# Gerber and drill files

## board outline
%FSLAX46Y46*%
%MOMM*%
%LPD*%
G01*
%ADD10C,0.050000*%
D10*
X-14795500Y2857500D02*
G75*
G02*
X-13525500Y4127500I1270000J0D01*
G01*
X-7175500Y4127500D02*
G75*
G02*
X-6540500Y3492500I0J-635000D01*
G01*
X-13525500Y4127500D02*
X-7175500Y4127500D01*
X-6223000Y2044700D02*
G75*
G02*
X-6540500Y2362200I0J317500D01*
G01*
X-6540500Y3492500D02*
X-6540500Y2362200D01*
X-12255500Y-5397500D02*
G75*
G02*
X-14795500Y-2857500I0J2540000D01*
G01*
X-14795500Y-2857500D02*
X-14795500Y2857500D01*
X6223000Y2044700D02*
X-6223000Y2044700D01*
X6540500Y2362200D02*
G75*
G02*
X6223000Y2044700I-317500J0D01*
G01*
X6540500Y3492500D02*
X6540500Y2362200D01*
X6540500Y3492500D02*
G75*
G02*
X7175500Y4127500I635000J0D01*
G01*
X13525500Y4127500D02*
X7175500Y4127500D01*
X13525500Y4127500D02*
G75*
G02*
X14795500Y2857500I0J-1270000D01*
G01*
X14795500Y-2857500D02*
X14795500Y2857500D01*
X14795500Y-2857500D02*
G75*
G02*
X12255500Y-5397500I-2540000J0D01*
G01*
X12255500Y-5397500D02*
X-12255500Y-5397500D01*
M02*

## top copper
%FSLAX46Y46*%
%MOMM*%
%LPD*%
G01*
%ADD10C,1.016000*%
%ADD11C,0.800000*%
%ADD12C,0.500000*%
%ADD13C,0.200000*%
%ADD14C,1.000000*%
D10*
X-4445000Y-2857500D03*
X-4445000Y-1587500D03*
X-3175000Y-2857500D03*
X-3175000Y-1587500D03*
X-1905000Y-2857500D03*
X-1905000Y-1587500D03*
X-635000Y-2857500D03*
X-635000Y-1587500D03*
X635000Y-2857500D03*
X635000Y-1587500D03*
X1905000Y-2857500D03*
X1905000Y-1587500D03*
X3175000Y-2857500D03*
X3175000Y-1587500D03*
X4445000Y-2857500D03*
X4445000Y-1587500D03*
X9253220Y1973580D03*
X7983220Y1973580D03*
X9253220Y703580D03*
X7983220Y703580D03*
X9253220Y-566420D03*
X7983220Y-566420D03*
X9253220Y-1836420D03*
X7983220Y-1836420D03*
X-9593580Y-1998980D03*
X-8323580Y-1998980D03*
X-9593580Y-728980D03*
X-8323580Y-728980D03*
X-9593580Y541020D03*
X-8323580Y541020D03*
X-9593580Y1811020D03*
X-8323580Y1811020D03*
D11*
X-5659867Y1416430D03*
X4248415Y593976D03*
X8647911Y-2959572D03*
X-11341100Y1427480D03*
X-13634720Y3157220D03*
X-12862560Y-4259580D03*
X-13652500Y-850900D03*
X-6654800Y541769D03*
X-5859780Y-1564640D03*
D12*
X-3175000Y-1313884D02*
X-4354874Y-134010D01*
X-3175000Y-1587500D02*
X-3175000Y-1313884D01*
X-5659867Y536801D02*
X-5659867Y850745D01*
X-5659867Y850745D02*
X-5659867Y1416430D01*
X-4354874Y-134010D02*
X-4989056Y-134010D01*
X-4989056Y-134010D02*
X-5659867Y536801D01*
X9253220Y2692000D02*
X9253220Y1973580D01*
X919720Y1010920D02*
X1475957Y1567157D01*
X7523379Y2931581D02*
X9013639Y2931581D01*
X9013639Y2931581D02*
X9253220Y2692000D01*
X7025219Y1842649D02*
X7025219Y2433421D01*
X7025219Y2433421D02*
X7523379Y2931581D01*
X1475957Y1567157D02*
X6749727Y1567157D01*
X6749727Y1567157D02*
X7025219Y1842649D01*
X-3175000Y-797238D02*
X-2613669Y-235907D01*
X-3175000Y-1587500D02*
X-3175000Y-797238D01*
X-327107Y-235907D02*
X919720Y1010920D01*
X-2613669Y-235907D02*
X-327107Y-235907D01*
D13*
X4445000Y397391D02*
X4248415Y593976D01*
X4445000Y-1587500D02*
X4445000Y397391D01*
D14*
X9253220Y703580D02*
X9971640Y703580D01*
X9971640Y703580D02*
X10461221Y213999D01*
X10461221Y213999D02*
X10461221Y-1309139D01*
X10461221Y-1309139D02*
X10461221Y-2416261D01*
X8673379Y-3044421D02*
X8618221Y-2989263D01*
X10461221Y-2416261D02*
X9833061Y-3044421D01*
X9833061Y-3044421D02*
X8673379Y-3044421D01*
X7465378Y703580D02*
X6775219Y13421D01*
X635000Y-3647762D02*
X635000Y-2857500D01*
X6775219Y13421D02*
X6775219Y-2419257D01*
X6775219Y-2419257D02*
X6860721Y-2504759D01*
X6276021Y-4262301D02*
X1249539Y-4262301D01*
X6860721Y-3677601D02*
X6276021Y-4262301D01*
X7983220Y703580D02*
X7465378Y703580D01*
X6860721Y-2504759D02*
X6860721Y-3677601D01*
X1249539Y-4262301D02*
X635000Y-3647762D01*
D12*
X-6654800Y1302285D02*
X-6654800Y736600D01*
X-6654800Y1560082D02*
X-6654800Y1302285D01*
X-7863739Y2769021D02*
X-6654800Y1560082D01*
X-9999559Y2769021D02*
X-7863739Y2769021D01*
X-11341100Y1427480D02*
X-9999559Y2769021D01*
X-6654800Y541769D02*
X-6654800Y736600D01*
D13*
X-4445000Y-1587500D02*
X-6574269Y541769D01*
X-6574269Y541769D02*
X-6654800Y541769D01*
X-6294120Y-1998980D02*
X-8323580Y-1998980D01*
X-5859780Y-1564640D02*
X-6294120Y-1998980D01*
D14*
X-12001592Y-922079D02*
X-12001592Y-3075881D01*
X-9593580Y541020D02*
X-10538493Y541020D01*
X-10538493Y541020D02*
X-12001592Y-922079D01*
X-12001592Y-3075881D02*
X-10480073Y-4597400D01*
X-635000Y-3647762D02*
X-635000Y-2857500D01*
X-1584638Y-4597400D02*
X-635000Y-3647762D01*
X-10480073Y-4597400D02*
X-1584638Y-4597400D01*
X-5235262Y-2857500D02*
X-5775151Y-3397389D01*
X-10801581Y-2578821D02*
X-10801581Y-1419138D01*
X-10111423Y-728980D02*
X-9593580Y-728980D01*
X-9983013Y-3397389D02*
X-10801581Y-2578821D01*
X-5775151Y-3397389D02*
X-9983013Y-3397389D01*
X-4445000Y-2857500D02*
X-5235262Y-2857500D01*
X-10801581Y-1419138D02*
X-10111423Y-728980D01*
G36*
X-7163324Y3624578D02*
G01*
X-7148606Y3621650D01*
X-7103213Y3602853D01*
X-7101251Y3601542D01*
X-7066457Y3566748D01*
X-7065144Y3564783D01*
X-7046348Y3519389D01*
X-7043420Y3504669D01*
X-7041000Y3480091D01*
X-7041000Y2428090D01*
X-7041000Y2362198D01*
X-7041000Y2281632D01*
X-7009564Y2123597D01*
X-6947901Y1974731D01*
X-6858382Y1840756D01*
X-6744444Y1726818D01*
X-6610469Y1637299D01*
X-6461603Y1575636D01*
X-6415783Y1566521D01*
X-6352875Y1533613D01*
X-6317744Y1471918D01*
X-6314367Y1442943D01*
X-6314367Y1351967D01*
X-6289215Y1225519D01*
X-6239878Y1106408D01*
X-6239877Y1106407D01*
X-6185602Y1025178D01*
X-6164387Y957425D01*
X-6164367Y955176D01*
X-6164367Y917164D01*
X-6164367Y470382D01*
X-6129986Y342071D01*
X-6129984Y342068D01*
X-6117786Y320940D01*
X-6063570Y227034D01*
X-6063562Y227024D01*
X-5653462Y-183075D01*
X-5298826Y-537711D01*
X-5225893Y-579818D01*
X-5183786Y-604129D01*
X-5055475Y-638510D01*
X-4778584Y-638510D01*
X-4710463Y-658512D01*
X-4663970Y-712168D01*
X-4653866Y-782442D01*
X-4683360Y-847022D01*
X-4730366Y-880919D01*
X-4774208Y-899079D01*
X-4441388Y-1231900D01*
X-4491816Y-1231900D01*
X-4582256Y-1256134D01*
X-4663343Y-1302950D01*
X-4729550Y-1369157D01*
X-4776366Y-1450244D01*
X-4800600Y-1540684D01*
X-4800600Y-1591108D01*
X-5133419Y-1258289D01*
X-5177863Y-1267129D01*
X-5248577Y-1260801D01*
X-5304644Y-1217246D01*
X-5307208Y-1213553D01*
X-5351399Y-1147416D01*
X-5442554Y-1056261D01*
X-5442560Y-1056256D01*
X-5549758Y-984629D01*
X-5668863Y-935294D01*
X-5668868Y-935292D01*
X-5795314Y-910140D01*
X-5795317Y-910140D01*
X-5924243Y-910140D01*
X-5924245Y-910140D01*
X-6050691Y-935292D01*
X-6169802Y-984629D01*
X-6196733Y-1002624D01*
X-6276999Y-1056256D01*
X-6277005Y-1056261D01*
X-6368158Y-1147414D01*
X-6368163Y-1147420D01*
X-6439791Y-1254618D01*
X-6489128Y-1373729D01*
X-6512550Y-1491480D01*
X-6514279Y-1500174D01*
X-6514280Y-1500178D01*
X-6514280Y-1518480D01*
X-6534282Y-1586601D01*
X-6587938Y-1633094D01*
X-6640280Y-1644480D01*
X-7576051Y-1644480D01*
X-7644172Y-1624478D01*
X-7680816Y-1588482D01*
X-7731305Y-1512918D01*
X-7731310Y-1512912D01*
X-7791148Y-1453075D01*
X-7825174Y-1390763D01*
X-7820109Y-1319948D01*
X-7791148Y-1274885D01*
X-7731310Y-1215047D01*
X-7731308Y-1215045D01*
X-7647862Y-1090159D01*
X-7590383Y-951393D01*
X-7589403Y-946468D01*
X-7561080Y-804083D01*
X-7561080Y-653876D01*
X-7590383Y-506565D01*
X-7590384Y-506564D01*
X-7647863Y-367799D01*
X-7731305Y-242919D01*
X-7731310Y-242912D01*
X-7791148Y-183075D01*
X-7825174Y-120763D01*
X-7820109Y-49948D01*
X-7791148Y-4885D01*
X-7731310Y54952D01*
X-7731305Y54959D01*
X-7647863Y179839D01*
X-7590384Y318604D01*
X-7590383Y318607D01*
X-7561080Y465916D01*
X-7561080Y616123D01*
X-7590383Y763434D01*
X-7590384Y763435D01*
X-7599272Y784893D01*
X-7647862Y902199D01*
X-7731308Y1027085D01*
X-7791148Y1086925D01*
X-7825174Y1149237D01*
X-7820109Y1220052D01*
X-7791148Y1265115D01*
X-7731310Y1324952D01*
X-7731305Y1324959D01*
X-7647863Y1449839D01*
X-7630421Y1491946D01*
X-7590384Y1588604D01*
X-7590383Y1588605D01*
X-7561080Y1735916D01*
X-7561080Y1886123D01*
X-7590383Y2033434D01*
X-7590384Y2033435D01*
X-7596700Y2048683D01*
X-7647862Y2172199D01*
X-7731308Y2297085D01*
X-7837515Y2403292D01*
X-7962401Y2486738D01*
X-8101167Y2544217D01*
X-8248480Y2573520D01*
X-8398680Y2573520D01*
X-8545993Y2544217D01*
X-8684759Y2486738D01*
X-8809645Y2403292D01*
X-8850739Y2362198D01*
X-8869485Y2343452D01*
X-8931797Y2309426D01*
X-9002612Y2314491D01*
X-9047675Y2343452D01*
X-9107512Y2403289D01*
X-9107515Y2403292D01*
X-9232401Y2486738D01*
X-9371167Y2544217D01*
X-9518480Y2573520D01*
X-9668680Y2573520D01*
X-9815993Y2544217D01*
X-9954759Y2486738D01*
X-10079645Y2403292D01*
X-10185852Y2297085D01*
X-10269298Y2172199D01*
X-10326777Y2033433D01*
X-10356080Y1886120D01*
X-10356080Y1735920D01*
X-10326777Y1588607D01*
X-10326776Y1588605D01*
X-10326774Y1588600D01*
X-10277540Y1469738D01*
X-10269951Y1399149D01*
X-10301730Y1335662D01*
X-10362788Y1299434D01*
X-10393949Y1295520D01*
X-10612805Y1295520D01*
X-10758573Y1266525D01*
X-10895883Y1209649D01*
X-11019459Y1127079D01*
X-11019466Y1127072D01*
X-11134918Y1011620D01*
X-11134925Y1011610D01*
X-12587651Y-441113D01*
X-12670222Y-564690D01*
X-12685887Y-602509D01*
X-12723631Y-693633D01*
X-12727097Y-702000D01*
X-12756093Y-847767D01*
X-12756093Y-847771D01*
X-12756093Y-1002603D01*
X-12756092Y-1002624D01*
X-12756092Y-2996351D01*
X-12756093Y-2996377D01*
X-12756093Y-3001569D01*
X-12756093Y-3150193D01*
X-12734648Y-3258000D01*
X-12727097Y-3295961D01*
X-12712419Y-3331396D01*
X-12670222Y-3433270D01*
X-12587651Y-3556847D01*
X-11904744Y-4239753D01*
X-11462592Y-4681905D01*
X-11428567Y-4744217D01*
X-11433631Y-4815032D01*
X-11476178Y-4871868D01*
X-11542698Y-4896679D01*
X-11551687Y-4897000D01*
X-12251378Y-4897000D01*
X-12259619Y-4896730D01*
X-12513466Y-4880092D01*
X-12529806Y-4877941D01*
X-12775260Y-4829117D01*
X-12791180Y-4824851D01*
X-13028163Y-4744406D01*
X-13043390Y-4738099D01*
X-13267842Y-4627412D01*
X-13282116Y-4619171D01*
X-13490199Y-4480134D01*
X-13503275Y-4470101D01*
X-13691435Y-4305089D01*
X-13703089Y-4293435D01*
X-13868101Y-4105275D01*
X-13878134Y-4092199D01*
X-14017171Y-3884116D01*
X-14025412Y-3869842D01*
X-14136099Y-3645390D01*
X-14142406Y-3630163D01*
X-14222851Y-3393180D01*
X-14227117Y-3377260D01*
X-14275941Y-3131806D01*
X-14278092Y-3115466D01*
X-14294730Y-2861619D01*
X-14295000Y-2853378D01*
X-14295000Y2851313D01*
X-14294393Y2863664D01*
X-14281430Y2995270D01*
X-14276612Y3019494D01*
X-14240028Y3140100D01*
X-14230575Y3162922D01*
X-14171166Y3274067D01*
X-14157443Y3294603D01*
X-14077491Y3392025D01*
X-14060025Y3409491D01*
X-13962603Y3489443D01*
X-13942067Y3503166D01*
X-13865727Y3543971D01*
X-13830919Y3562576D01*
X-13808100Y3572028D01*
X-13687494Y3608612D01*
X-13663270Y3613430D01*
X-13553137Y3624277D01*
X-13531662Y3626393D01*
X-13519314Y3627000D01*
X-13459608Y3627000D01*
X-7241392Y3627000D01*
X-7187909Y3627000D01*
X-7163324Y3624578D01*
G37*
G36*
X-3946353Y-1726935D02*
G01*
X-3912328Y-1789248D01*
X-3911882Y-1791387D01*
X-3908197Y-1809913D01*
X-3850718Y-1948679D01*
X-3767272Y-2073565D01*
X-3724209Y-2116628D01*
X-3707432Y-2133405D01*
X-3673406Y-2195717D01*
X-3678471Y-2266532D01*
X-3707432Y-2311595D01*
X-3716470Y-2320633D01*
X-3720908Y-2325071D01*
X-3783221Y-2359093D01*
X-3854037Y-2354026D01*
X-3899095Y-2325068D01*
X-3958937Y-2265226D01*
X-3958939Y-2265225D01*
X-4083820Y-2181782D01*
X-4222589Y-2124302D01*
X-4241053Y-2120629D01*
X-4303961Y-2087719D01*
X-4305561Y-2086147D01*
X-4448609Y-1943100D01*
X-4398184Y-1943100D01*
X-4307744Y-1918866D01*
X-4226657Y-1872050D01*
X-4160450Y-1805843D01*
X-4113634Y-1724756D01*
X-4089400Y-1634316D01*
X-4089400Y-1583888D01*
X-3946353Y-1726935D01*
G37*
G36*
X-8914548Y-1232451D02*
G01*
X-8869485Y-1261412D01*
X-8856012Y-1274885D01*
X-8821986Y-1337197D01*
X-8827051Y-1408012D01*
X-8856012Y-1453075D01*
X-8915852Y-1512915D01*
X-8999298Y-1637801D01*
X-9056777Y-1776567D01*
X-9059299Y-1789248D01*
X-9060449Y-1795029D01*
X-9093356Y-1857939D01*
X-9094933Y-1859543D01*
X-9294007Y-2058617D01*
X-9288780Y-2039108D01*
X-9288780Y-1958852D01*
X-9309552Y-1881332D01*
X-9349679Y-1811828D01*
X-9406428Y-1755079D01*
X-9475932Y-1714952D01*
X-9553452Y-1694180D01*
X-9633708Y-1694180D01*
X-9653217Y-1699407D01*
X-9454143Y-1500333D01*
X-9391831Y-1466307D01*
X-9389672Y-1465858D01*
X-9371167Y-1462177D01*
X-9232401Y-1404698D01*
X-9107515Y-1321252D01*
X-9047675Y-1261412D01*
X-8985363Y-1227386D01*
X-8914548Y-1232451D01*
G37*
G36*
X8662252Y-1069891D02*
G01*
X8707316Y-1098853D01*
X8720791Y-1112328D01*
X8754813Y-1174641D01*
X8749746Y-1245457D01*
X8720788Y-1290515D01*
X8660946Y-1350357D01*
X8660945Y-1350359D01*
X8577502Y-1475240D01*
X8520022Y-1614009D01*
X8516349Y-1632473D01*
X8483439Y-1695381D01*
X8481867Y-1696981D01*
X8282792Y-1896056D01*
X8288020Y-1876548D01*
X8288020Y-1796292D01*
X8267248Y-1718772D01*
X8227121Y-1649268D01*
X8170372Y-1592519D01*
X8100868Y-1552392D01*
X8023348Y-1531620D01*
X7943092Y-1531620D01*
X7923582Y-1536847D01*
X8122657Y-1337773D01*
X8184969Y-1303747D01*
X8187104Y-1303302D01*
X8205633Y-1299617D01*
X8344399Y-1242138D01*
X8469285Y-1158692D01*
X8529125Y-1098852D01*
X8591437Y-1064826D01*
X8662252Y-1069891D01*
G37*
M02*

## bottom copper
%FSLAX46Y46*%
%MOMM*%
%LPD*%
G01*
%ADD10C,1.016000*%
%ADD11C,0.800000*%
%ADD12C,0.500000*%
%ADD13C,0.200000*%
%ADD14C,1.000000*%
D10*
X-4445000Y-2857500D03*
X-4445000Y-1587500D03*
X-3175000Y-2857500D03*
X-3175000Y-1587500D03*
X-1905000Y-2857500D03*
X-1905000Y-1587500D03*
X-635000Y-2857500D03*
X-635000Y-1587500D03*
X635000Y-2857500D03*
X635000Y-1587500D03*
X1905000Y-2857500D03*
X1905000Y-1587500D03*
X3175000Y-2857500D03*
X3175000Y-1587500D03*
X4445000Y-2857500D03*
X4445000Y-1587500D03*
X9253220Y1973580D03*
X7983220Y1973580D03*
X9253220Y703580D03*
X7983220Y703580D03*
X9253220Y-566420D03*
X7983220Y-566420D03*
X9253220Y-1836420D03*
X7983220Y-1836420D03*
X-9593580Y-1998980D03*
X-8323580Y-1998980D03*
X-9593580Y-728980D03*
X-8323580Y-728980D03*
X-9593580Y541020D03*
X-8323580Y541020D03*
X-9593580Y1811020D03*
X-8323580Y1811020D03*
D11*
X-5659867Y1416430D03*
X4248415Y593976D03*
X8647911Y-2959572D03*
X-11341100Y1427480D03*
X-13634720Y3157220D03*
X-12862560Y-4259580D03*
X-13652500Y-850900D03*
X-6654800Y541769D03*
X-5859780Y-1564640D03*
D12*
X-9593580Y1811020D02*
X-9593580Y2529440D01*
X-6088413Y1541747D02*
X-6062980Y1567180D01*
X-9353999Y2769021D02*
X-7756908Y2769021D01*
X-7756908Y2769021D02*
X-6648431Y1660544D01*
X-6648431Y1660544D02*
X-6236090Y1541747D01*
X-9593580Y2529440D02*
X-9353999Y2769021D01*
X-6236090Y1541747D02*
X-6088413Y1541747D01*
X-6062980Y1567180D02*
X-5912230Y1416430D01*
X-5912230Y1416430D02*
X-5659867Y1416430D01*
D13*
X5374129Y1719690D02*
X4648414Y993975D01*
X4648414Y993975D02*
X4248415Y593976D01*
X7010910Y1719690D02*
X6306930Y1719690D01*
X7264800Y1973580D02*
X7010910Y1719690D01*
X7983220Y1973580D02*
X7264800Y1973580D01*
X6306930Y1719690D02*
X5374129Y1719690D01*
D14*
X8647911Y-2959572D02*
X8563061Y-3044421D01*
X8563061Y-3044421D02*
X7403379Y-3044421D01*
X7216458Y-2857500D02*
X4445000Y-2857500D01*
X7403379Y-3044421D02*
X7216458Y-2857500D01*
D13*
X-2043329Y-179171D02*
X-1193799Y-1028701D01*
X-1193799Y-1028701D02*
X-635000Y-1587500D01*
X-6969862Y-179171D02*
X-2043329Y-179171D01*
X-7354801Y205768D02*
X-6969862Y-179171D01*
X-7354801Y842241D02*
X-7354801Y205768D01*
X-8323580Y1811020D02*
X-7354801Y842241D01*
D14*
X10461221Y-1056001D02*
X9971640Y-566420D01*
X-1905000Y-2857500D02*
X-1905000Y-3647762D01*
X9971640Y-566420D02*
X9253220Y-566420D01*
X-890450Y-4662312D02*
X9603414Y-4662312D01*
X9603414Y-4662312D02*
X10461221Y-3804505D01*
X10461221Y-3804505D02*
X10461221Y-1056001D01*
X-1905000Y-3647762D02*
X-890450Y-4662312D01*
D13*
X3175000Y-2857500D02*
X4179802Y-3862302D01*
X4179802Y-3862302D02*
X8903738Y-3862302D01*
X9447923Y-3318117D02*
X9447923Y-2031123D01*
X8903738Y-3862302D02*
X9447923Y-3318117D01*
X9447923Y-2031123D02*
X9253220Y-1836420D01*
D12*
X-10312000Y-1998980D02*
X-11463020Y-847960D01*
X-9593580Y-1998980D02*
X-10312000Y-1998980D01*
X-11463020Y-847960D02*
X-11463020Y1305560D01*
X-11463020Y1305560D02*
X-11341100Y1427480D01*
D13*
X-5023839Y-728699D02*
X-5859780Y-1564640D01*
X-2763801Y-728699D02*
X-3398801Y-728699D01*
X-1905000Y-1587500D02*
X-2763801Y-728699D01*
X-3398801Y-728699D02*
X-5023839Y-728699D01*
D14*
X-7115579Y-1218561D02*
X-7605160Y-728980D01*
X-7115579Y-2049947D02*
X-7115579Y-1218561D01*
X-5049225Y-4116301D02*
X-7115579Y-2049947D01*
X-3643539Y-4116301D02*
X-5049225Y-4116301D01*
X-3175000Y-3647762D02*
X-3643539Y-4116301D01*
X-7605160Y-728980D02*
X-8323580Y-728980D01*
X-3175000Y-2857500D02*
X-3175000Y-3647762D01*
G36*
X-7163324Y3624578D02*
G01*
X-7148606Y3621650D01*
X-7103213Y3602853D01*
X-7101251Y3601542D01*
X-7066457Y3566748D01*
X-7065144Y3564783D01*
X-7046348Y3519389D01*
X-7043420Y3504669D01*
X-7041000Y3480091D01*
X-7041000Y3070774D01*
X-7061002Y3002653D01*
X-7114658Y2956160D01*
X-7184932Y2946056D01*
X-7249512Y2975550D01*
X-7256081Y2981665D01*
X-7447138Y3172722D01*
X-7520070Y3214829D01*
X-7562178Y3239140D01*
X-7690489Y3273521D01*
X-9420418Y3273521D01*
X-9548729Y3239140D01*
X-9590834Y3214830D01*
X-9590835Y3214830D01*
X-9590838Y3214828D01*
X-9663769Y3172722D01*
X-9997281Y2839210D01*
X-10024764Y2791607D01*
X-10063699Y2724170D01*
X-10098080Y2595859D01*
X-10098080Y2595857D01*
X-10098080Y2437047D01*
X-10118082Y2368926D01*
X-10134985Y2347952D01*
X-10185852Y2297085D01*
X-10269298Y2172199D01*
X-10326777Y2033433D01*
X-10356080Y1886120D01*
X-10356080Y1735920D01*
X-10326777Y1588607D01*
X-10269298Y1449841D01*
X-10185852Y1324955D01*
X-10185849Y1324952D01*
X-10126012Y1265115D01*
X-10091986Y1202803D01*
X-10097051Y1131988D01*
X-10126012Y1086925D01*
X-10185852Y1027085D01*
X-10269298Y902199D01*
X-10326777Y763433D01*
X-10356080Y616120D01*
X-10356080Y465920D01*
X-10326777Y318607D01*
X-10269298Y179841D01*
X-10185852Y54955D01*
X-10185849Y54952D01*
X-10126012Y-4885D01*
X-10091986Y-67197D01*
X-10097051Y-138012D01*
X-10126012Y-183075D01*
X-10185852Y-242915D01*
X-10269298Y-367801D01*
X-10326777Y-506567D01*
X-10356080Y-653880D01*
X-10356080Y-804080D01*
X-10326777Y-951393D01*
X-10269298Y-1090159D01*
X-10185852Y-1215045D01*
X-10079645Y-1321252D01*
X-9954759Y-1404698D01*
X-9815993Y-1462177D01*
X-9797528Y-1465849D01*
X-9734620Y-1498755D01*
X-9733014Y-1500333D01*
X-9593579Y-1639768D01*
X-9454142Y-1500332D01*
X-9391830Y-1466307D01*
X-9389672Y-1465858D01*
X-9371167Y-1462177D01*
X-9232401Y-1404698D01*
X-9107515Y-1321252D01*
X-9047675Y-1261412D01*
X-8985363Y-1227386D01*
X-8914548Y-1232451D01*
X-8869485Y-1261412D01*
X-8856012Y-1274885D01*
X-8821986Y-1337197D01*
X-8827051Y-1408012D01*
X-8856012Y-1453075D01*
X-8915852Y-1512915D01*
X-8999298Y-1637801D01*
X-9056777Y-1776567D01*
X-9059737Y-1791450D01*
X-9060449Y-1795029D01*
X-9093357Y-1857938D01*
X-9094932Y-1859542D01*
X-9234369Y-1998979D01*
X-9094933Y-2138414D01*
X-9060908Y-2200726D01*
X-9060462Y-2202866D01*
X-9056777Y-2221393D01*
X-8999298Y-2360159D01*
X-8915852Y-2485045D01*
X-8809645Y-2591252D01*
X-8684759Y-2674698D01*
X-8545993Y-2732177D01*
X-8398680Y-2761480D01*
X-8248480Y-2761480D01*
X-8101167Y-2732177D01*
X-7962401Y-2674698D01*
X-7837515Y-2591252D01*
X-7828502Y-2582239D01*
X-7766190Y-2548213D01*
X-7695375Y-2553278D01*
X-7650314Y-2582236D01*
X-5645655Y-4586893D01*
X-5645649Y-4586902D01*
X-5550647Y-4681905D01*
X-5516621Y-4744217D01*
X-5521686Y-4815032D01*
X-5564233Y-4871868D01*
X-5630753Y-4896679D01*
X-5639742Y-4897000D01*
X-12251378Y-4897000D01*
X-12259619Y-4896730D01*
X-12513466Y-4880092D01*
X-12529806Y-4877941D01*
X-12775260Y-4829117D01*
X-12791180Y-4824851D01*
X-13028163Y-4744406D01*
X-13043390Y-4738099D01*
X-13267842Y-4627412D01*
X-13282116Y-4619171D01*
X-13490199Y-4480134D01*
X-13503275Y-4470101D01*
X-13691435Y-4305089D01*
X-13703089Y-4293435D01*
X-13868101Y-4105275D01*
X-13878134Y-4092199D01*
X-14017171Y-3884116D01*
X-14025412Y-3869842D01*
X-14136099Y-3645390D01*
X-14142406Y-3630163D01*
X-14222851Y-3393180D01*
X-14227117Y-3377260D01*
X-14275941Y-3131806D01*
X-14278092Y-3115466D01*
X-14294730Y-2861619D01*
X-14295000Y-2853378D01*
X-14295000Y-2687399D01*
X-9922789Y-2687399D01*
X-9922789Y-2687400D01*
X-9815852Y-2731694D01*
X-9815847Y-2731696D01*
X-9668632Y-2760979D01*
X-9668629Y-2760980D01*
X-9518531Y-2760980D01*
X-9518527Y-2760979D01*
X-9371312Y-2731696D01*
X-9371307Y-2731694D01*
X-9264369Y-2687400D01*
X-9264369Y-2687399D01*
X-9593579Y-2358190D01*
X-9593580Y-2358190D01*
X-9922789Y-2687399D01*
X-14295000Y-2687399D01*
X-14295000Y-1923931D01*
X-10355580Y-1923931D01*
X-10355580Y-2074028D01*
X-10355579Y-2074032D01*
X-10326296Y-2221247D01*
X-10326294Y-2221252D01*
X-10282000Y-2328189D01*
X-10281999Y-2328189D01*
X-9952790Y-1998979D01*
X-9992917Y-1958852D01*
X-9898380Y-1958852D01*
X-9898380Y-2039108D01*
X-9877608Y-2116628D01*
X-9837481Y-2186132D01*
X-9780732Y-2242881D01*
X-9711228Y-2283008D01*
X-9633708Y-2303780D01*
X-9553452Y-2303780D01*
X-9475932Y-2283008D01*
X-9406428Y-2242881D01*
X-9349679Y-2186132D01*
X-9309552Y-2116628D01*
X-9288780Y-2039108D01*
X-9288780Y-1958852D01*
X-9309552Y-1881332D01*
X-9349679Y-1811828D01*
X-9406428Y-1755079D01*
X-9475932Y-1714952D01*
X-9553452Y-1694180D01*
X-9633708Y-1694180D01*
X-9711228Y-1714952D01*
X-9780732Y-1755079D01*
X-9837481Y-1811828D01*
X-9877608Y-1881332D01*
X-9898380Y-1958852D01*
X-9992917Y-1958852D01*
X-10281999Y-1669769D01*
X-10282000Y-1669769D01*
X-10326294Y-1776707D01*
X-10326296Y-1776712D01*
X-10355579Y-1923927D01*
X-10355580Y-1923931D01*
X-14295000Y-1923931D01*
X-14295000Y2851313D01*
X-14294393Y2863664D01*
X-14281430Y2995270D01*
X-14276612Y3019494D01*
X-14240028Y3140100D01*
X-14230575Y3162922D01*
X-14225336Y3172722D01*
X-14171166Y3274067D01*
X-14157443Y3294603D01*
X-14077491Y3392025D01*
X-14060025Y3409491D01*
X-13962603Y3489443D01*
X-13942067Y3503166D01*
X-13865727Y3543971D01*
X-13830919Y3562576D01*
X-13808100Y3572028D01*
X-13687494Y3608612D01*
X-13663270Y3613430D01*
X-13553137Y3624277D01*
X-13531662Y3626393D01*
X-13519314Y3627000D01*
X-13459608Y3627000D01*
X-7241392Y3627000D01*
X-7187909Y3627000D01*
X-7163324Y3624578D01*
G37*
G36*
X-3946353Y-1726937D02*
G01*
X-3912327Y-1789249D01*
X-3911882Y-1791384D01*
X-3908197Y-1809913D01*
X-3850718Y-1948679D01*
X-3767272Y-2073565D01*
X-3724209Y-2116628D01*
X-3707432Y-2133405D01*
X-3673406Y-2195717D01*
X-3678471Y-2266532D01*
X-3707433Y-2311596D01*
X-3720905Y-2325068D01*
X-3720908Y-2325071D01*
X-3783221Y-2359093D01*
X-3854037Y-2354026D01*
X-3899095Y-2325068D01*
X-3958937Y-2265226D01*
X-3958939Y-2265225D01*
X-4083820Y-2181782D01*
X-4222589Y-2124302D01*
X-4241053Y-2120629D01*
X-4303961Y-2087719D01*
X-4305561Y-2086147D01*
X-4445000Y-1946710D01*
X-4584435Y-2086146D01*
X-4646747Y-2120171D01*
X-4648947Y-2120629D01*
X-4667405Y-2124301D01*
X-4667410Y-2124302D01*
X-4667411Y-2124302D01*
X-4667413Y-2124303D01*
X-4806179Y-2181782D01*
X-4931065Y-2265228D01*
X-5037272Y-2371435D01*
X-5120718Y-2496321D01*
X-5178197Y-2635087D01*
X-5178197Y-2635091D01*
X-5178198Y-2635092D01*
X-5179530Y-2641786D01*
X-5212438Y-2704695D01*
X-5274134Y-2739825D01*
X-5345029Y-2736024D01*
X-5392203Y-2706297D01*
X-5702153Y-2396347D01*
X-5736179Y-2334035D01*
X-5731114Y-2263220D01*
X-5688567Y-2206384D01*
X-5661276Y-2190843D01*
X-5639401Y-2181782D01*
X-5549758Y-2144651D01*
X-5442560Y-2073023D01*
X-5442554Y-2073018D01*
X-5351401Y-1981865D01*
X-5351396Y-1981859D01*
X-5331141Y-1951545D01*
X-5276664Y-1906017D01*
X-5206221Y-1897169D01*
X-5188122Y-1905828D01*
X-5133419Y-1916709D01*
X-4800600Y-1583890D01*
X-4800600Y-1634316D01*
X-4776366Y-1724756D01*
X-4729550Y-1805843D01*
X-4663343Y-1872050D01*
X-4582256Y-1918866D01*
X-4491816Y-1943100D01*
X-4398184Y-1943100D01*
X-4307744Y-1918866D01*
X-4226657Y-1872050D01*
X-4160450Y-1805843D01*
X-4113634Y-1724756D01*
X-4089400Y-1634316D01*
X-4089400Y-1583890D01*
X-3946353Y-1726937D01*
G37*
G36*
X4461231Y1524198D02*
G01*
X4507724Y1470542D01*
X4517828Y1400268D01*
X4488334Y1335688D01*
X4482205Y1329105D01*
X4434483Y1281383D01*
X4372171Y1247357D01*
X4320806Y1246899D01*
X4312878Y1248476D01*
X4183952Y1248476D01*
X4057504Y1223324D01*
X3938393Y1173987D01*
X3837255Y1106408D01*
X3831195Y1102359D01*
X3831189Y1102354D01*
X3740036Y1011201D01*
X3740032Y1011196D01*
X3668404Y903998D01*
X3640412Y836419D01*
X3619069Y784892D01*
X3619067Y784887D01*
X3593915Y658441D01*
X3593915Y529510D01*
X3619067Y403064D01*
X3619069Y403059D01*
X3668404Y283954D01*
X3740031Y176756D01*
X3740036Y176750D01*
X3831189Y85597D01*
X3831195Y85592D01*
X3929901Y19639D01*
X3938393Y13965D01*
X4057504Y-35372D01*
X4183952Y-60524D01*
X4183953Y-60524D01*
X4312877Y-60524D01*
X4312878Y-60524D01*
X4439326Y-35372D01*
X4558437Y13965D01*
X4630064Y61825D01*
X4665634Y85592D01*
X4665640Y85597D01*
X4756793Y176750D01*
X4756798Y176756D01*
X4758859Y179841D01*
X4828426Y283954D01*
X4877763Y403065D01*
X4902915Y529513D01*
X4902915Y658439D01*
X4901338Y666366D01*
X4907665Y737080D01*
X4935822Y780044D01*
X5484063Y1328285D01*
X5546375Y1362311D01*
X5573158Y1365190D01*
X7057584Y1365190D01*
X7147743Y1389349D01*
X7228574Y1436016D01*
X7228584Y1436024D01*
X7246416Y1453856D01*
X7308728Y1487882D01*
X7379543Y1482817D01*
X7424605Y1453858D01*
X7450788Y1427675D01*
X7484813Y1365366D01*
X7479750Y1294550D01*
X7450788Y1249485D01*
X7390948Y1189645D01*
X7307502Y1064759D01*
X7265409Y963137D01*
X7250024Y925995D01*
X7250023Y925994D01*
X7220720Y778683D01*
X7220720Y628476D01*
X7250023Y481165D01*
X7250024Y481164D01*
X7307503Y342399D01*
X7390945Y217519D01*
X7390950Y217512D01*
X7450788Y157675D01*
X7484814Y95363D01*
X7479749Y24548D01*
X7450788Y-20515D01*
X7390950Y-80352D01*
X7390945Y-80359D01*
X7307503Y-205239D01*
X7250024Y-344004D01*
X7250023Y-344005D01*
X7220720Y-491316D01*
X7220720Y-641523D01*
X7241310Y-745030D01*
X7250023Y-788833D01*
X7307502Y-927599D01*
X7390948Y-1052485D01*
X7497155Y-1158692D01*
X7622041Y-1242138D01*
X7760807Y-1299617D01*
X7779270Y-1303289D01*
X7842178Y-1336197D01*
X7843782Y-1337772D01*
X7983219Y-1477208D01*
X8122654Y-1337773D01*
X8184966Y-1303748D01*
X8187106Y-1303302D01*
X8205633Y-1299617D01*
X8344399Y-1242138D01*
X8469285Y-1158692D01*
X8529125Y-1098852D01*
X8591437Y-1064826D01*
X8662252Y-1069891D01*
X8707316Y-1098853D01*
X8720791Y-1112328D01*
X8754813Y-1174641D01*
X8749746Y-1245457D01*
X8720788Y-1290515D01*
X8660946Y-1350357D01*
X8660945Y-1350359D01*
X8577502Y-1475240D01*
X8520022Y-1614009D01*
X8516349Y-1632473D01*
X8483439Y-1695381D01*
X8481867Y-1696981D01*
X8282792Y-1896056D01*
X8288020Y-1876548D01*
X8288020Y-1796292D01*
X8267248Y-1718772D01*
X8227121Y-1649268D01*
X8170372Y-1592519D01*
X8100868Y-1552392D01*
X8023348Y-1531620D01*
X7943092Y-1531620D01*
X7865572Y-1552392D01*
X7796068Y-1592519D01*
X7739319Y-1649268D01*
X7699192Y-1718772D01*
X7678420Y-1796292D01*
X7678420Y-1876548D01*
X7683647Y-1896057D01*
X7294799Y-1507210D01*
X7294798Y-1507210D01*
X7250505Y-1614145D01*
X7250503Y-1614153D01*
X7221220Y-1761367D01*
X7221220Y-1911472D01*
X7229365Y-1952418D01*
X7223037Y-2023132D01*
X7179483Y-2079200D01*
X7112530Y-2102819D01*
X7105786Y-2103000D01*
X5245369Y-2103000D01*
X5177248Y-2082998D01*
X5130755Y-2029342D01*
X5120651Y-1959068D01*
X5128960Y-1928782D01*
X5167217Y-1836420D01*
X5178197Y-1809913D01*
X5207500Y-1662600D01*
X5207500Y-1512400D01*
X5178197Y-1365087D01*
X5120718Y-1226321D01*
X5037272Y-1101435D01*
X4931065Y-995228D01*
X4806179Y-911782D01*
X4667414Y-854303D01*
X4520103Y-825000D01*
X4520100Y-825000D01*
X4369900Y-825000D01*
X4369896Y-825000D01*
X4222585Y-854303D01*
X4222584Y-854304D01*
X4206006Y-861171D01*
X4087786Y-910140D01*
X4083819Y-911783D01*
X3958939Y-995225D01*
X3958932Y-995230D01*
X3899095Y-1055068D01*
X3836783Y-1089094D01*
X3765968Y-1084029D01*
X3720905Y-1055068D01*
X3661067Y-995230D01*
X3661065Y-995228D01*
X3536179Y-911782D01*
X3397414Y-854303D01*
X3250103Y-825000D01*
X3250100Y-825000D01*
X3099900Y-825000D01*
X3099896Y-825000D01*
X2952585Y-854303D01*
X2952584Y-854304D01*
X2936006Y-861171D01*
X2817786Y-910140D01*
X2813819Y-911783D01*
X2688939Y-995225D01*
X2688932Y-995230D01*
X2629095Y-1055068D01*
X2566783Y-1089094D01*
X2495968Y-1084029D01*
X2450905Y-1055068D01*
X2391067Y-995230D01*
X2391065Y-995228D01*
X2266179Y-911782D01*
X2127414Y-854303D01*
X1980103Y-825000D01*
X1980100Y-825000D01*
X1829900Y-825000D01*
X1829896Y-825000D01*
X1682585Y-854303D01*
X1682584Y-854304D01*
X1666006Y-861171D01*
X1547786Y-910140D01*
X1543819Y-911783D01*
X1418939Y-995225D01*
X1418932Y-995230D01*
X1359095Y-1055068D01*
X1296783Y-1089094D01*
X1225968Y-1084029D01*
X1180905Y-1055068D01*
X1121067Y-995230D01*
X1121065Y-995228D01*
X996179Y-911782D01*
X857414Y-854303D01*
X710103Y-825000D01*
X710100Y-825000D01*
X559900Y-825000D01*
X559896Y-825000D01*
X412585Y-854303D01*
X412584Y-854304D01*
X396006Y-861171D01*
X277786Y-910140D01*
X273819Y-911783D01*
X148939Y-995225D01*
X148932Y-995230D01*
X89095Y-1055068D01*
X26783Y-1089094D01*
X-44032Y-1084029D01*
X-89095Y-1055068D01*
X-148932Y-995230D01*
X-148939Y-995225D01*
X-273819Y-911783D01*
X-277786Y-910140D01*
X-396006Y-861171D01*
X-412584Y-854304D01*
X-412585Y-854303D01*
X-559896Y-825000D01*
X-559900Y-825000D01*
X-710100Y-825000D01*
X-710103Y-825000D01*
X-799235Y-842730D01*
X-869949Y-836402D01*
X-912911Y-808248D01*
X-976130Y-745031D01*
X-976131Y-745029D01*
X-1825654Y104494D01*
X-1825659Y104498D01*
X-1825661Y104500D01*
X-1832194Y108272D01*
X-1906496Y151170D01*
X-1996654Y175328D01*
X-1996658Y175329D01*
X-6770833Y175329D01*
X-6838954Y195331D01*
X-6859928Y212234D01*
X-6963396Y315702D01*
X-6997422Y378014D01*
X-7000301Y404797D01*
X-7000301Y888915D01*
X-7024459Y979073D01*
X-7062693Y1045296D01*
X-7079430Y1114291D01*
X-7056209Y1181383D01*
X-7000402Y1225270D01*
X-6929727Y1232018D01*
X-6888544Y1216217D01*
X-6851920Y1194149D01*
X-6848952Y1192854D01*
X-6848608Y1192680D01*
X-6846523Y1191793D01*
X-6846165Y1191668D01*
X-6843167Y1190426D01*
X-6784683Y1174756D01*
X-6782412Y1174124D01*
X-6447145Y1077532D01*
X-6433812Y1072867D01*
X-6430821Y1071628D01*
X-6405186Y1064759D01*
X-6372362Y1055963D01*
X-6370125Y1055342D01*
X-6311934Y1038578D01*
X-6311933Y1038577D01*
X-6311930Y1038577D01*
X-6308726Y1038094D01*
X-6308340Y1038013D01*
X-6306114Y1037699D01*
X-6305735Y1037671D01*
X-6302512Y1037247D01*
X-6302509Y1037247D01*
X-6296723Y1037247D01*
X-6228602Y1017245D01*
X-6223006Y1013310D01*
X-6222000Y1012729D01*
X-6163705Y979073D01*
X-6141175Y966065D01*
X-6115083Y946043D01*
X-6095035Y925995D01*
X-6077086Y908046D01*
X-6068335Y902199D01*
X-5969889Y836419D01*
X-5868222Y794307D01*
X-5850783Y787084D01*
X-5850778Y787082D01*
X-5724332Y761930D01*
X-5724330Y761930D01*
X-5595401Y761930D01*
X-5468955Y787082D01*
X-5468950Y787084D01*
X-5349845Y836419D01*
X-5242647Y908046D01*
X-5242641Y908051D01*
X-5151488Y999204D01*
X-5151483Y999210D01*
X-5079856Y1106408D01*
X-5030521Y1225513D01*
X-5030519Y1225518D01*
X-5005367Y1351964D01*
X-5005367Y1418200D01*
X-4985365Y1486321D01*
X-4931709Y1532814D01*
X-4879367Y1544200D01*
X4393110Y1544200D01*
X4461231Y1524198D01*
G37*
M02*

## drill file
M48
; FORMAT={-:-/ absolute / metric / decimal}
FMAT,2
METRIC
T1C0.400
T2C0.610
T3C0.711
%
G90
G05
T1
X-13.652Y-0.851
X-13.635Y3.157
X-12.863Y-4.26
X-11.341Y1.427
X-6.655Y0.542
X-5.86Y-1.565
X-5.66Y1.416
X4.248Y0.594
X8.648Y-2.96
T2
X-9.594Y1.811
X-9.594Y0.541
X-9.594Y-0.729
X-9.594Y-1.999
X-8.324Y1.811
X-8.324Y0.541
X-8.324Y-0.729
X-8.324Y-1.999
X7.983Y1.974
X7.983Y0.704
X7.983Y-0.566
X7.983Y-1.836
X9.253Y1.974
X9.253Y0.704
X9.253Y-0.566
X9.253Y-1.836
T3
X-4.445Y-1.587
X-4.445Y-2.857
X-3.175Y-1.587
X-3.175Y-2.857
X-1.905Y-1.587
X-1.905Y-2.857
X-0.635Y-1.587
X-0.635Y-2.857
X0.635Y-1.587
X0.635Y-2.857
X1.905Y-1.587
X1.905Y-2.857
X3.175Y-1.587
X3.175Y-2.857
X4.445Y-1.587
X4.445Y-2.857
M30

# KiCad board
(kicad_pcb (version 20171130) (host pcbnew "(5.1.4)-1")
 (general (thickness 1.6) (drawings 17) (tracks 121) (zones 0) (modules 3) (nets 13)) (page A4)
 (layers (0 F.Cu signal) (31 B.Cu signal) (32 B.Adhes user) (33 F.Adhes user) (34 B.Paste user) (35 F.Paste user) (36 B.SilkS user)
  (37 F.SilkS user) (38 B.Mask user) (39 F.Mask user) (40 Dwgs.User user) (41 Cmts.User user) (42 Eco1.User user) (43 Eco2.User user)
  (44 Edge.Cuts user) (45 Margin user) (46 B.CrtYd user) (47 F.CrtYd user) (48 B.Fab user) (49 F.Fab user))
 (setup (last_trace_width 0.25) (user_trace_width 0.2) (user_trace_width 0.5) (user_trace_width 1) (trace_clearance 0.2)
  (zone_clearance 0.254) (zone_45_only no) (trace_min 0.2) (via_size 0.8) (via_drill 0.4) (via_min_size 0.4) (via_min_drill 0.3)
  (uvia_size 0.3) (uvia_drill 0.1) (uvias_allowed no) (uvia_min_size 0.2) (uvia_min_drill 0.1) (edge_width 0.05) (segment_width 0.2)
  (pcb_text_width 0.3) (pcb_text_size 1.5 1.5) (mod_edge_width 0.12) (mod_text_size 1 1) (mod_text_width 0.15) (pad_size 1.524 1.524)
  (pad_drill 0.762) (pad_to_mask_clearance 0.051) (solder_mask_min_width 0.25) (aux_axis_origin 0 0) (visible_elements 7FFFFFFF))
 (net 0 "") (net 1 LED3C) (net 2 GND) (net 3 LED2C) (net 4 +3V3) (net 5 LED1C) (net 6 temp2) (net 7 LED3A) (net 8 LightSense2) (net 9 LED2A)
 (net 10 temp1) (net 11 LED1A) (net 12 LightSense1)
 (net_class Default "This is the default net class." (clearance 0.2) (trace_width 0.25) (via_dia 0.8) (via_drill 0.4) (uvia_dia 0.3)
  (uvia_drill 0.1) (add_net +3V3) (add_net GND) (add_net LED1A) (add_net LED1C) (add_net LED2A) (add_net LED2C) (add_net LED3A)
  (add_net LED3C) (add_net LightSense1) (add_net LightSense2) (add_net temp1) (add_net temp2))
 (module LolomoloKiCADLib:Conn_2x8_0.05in (layer F.Cu) (at 4.445 1.5875 270)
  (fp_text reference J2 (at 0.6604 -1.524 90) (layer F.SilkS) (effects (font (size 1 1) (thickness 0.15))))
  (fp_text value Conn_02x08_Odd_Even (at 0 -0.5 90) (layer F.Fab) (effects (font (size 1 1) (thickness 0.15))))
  (pad 16 thru_hole circle (at 1.27 8.89 270) (size 1.016 1.016) (drill 0.7112) (layers *.Cu *.Mask) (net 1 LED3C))
  (pad 15 thru_hole circle (at 0 8.89 270) (size 1.016 1.016) (drill 0.7112) (layers *.Cu *.Mask) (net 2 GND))
  (pad 14 thru_hole circle (at 1.27 7.62 270) (size 1.016 1.016) (drill 0.7112) (layers *.Cu *.Mask) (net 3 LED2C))
  (pad 13 thru_hole circle (at 0 7.62 270) (size 1.016 1.016) (drill 0.7112) (layers *.Cu *.Mask) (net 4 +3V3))
  (pad 12 thru_hole circle (at 1.27 6.35 270) (size 1.016 1.016) (drill 0.7112) (layers *.Cu *.Mask) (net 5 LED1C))
  (pad 11 thru_hole circle (at 0 6.35 270) (size 1.016 1.016) (drill 0.7112) (layers *.Cu *.Mask) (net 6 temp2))
  (pad 10 thru_hole circle (at 1.27 5.08 270) (size 1.016 1.016) (drill 0.7112) (layers *.Cu *.Mask) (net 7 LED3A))
  (pad 9 thru_hole circle (at 0 5.08 270) (size 1.016 1.016) (drill 0.7112) (layers *.Cu *.Mask) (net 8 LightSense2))
  (pad 8 thru_hole circle (at 1.27 3.81 270) (size 1.016 1.016) (drill 0.7112) (layers *.Cu *.Mask) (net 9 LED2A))
  (pad 7 thru_hole circle (at 0 3.81 270) (size 1.016 1.016) (drill 0.7112) (layers *.Cu *.Mask))
  (pad 6 thru_hole circle (at 1.27 2.54 270) (size 1.016 1.016) (drill 0.7112) (layers *.Cu *.Mask))
  (pad 5 thru_hole circle (at 0 2.54 270) (size 1.016 1.016) (drill 0.7112) (layers *.Cu *.Mask))
  (pad 4 thru_hole circle (at 1.27 1.27 270) (size 1.016 1.016) (drill 0.7112) (layers *.Cu *.Mask) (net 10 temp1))
  (pad 3 thru_hole circle (at 0 1.27 270) (size 1.016 1.016) (drill 0.7112) (layers *.Cu *.Mask))
  (pad 2 thru_hole circle (at 1.27 0 270) (size 1.016 1.016) (drill 0.7112) (layers *.Cu *.Mask) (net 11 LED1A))
  (pad 1 thru_hole circle (at 0 0 270) (size 1.016 1.016) (drill 0.7112) (layers *.Cu *.Mask) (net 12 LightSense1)))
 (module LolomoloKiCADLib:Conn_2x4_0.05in (layer B.Cu) (at 9.25322 -1.97358 180)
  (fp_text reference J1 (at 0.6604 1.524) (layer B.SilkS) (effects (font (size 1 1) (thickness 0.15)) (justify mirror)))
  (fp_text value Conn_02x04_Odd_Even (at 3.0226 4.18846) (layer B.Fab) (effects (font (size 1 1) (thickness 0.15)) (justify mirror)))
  (pad 1 thru_hole circle (at 0 0 180) (size 1.016 1.016) (drill 0.6096) (layers *.Cu *.Mask) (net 4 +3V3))
  (pad 2 thru_hole circle (at 1.27 0 180) (size 1.016 1.016) (drill 0.6096) (layers *.Cu *.Mask) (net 12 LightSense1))
  (pad 3 thru_hole circle (at 0 -1.27 180) (size 1.016 1.016) (drill 0.6096) (layers *.Cu *.Mask) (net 11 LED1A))
  (pad 4 thru_hole circle (at 1.27 -1.27 180) (size 1.016 1.016) (drill 0.6096) (layers *.Cu *.Mask) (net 9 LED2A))
  (pad 5 thru_hole circle (at 0 -2.54 180) (size 1.016 1.016) (drill 0.6096) (layers *.Cu *.Mask) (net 5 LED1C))
  (pad 6 thru_hole circle (at 1.27 -2.54 180) (size 1.016 1.016) (drill 0.6096) (layers *.Cu *.Mask))
  (pad 7 thru_hole circle (at 0 -3.81 180) (size 1.016 1.016) (drill 0.6096) (layers *.Cu *.Mask) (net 10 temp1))
  (pad 8 thru_hole circle (at 1.27 -3.81 180) (size 1.016 1.016) (drill 0.6096) (layers *.Cu *.Mask) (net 2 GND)))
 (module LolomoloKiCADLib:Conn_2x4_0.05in (layer B.Cu) (at -8.32358 -1.81102 180)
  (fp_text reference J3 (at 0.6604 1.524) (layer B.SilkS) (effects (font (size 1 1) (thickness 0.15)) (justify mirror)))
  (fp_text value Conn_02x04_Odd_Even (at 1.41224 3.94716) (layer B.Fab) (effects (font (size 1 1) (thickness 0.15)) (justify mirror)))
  (pad 8 thru_hole circle (at 1.27 -3.81 180) (size 1.016 1.016) (drill 0.6096) (layers *.Cu *.Mask) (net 2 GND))
  (pad 7 thru_hole circle (at 0 -3.81 180) (size 1.016 1.016) (drill 0.6096) (layers *.Cu *.Mask) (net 6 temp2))
  (pad 6 thru_hole circle (at 1.27 -2.54 180) (size 1.016 1.016) (drill 0.6096) (layers *.Cu *.Mask) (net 1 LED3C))
  (pad 5 thru_hole circle (at 0 -2.54 180) (size 1.016 1.016) (drill 0.6096) (layers *.Cu *.Mask) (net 3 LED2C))
  (pad 4 thru_hole circle (at 1.27 -1.27 180) (size 1.016 1.016) (drill 0.6096) (layers *.Cu *.Mask) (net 7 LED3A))
  (pad 3 thru_hole circle (at 0 -1.27 180) (size 1.016 1.016) (drill 0.6096) (layers *.Cu *.Mask))
  (pad 2 thru_hole circle (at 1.27 0 180) (size 1.016 1.016) (drill 0.6096) (layers *.Cu *.Mask) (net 4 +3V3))
  (pad 1 thru_hole circle (at 0 0 180) (size 1.016 1.016) (drill 0.6096) (layers *.Cu *.Mask) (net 8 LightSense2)))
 (gr_arc (start -13.5255 -2.8575) (end -14.7955 -2.8575) (angle 90) (layer Edge.Cuts) (width 0.05))
 (gr_arc (start -7.1755 -3.4925) (end -7.1755 -4.1275) (angle 90) (layer Edge.Cuts) (width 0.05))
 (gr_line (start -13.5255 -4.1275) (end -7.1755 -4.1275) (layer Edge.Cuts) (width 0.05))
 (gr_arc (start -6.223 -2.3622) (end -6.5405 -2.3622) (angle -90) (layer Edge.Cuts) (width 0.05))
 (gr_line (start -6.5405 -3.4925) (end -6.5405 -2.3622) (layer Edge.Cuts) (width 0.05))
 (gr_arc (start -12.2555 2.8575) (end -12.2555 5.3975) (angle 90) (layer Edge.Cuts) (width 0.05))
 (gr_line (start -14.7955 2.8575) (end -14.7955 -2.8575) (layer Edge.Cuts) (width 0.05))
 (gr_line (start 6.223 -2.0447) (end -6.223 -2.0447) (layer Edge.Cuts) (width 0.05))
 (gr_arc (start 6.223 -2.3622) (end 6.5405 -2.3622) (angle 90) (layer Edge.Cuts) (width 0.05))
 (gr_line (start 6.5405 -3.4925) (end 6.5405 -2.3622) (layer Edge.Cuts) (width 0.05))
 (gr_arc (start 7.1755 -3.4925) (end 7.1755 -4.1275) (angle -90) (layer Edge.Cuts) (width 0.05))
 (gr_line (start 13.5255 -4.1275) (end 7.1755 -4.1275) (layer Edge.Cuts) (width 0.05))
 (gr_arc (start 13.5255 -2.8575) (end 14.7955 -2.8575) (angle -90) (layer Edge.Cuts) (width 0.05))
 (gr_line (start 14.7955 2.8575) (end 14.7955 -2.8575) (layer Edge.Cuts) (width 0.05))
 (gr_arc (start 12.2555 2.8575) (end 12.2555 5.3975) (angle -90) (layer Edge.Cuts) (width 0.05))
 (gr_line (start 12.2555 5.3975) (end -12.2555 5.3975) (layer Edge.Cuts) (width 0.05))
 (segment (start -9.59358 -1.81102) (end -9.59358 -2.52944) (width 0.5) (layer B.Cu) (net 4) (status 10))
 (segment (start -6.088413 -1.541747) (end -6.06298 -1.56718) (width 0.5) (layer B.Cu) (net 4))
 (segment (start -9.353999 -2.769021) (end -7.756908 -2.769021) (width 0.5) (layer B.Cu) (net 4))
 (segment (start -7.756908 -2.769021) (end -6.648431 -1.660544) (width 0.5) (layer B.Cu) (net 4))
 (segment (start -6.648431 -1.660544) (end -6.23609 -1.541747) (width 0.5) (layer B.Cu) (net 4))
 (segment (start -9.59358 -2.52944) (end -9.353999 -2.769021) (width 0.5) (layer B.Cu) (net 4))
 (segment (start -6.23609 -1.541747) (end -6.088413 -1.541747) (width 0.5) (layer B.Cu) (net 4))
 (segment (start -3.175 1.313884) (end -4.354874 0.13401) (width 0.5) (layer F.Cu) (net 4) (status 10))
 (segment (start -6.06298 -1.56718) (end -5.91223 -1.41643) (width 0.5) (layer B.Cu) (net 4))
 (segment (start -3.175 1.5875) (end -3.175 1.313884) (width 0.5) (layer F.Cu) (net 4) (status 30))
 (segment (start -5.659867 -0.536801) (end -5.659867 -0.850745) (width 0.5) (layer F.Cu) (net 4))
 (segment (start -5.659867 -0.850745) (end -5.659867 -1.41643) (width 0.5) (layer F.Cu) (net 4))
 (segment (start -4.354874 0.13401) (end -4.989056 0.13401) (width 0.5) (layer F.Cu) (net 4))
 (segment (start -4.989056 0.13401) (end -5.659867 -0.536801) (width 0.5) (layer F.Cu) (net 4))
 (via (at -5.659867 -1.41643) (size 0.8) (drill 0.4) (layers F.Cu B.Cu) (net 4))
 (segment (start -5.91223 -1.41643) (end -5.659867 -1.41643) (width 0.5) (layer B.Cu) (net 4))
 (segment (start 9.25322 -2.692) (end 9.25322 -1.97358) (width 0.5) (layer F.Cu) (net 4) (status 20))
 (segment (start 0.91972 -1.01092) (end 1.475957 -1.567157) (width 0.5) (layer F.Cu) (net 4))
 (segment (start 7.523379 -2.931581) (end 9.013639 -2.931581) (width 0.5) (layer F.Cu) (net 4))
 (segment (start 9.013639 -2.931581) (end 9.25322 -2.692) (width 0.5) (layer F.Cu) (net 4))
 (segment (start 7.025219 -1.842649) (end 7.025219 -2.433421) (width 0.5) (layer F.Cu) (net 4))
 (segment (start 7.025219 -2.433421) (end 7.523379 -2.931581) (width 0.5) (layer F.Cu) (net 4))
 (segment (start 1.475957 -1.567157) (end 6.749727 -1.567157) (width 0.5) (layer F.Cu) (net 4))
 (segment (start 6.749727 -1.567157) (end 7.025219 -1.842649) (width 0.5) (layer F.Cu) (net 4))
 (segment (start -3.175 0.797238) (end -2.613669 0.235907) (width 0.5) (layer F.Cu) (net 4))
 (segment (start -3.175 1.5875) (end -3.175 0.797238) (width 0.5) (layer F.Cu) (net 4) (status 10))
 (segment (start -0.327107 0.235907) (end 0.91972 -1.01092) (width 0.5) (layer F.Cu) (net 4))
 (segment (start -2.613669 0.235907) (end -0.327107 0.235907) (width 0.5) (layer F.Cu) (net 4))
 (segment (start 4.445 -0.397391) (end 4.248415 -0.593976) (width 0.2) (layer F.Cu) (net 12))
 (segment (start 5.374129 -1.71969) (end 4.648414 -0.993975) (width 0.2) (layer B.Cu) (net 12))
 (via (at 4.248415 -0.593976) (size 0.8) (drill 0.4) (layers F.Cu B.Cu) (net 12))
 (segment (start 4.648414 -0.993975) (end 4.248415 -0.593976) (width 0.2) (layer B.Cu) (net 12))
 (segment (start 4.445 1.5875) (end 4.445 -0.397391) (width 0.2) (layer F.Cu) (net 12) (status 10))
 (segment (start 7.01091 -1.71969) (end 6.30693 -1.71969) (width 0.2) (layer B.Cu) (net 12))
 (segment (start 7.2648 -1.97358) (end 7.01091 -1.71969) (width 0.2) (layer B.Cu) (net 12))
 (segment (start 7.98322 -1.97358) (end 7.2648 -1.97358) (width 0.2) (layer B.Cu) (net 12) (status 10))
 (segment (start 6.30693 -1.71969) (end 5.374129 -1.71969) (width 0.2) (layer B.Cu) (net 12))
 (segment (start 9.25322 -0.70358) (end 9.97164 -0.70358) (width 1) (layer F.Cu) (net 11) (status 10))
 (segment (start 9.97164 -0.70358) (end 10.461221 -0.213999) (width 1) (layer F.Cu) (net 11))
 (via (at 8.647911 2.959572) (size 0.8) (drill 0.4) (layers F.Cu B.Cu) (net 11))
 (segment (start 10.461221 -0.213999) (end 10.461221 1.309139) (width 1) (layer F.Cu) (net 11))
 (segment (start 10.461221 1.309139) (end 10.461221 2.416261) (width 1) (layer F.Cu) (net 11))
 (segment (start 8.673379 3.044421) (end 8.618221 2.989263) (width 1) (layer F.Cu) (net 11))
 (segment (start 10.461221 2.416261) (end 9.833061 3.044421) (width 1) (layer F.Cu) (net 11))
 (segment (start 9.833061 3.044421) (end 8.673379 3.044421) (width 1) (layer F.Cu) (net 11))
 (segment (start 8.647911 2.959572) (end 8.563061 3.044421) (width 1) (layer B.Cu) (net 11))
 (segment (start 8.563061 3.044421) (end 7.403379 3.044421) (width 1) (layer B.Cu) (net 11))
 (segment (start 7.216458 2.8575) (end 4.445 2.8575) (width 1) (layer B.Cu) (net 11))
 (segment (start 7.403379 3.044421) (end 7.216458 2.8575) (width 1) (layer B.Cu) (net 11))
 (segment (start -2.043329 0.179171) (end -1.193799 1.028701) (width 0.2) (layer B.Cu) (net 8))
 (segment (start -1.193799 1.028701) (end -0.635 1.5875) (width 0.2) (layer B.Cu) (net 8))
 (segment (start -6.969862 0.179171) (end -2.043329 0.179171) (width 0.2) (layer B.Cu) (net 8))
 (segment (start -7.354801 -0.205768) (end -6.969862 0.179171) (width 0.2) (layer B.Cu) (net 8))
 (segment (start -7.354801 -0.842241) (end -7.354801 -0.205768) (width 0.2) (layer B.Cu) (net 8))
 (segment (start -8.32358 -1.81102) (end -7.354801 -0.842241) (width 0.2) (layer B.Cu) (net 8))
 (segment (start 10.461221 1.056001) (end 9.97164 0.56642) (width 1) (layer B.Cu) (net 5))
 (segment (start -1.905 2.8575) (end -1.905 3.647762) (width 1) (layer B.Cu) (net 5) (status 10))
 (segment (start 9.97164 0.56642) (end 9.25322 0.56642) (width 1) (layer B.Cu) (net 5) (status 20))
 (segment (start -0.89045 4.662312) (end 9.603414 4.662312) (width 1) (layer B.Cu) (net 5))
 (segment (start 9.603414 4.662312) (end 10.461221 3.804505) (width 1) (layer B.Cu) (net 5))
 (segment (start 10.461221 3.804505) (end 10.461221 1.056001) (width 1) (layer B.Cu) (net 5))
 (segment (start -1.905 3.647762) (end -0.89045 4.662312) (width 1) (layer B.Cu) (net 5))
 (segment (start 7.465378 -0.70358) (end 6.775219 -0.013421) (width 1) (layer F.Cu) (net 9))
 (segment (start 0.635 3.647762) (end 0.635 2.8575) (width 1) (layer F.Cu) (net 9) (status 20))
 (segment (start 6.775219 -0.013421) (end 6.775219 2.419257) (width 1) (layer F.Cu) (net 9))
 (segment (start 6.775219 2.419257) (end 6.860721 2.504759) (width 1) (layer F.Cu) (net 9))
 (segment (start 6.276021 4.262301) (end 1.249539 4.262301) (width 1) (layer F.Cu) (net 9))
 (segment (start 6.860721 3.677601) (end 6.276021 4.262301) (width 1) (layer F.Cu) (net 9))
 (segment (start 7.98322 -0.70358) (end 7.465378 -0.70358) (width 1) (layer F.Cu) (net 9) (status 10))
 (segment (start 6.860721 2.504759) (end 6.860721 3.677601) (width 1) (layer F.Cu) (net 9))
 (segment (start 1.249539 4.262301) (end 0.635 3.647762) (width 1) (layer F.Cu) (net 9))
 (segment (start 3.175 2.8575) (end 4.179802 3.862302) (width 0.2) (layer B.Cu) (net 10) (status 10))
 (segment (start 4.179802 3.862302) (end 8.903738 3.862302) (width 0.2) (layer B.Cu) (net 10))
 (segment (start 9.447923 3.318117) (end 9.447923 2.031123) (width 0.2) (layer B.Cu) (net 10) (status 20))
 (segment (start 8.903738 3.862302) (end 9.447923 3.318117) (width 0.2) (layer B.Cu) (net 10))
 (segment (start 9.447923 2.031123) (end 9.25322 1.83642) (width 0.2) (layer B.Cu) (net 10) (status 30))
 (segment (start -10.312 1.99898) (end -11.46302 0.84796) (width 0.5) (layer B.Cu) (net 2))
 (segment (start -9.59358 1.99898) (end -10.312 1.99898) (width 0.5) (layer B.Cu) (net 2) (status 10))
 (via (at -11.3411 -1.42748) (size 0.8) (drill 0.4) (layers F.Cu B.Cu) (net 2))
 (segment (start -11.46302 0.84796) (end -11.46302 -1.30556) (width 0.5) (layer B.Cu) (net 2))
 (segment (start -11.46302 -1.30556) (end -11.3411 -1.42748) (width 0.5) (layer B.Cu) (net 2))
 (segment (start -6.6548 -1.302285) (end -6.6548 -0.7366) (width 0.5) (layer F.Cu) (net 2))
 (segment (start -6.6548 -1.560082) (end -6.6548 -1.302285) (width 0.5) (layer F.Cu) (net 2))
 (segment (start -7.863739 -2.769021) (end -6.6548 -1.560082) (width 0.5) (layer F.Cu) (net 2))
 (segment (start -9.999559 -2.769021) (end -7.863739 -2.769021) (width 0.5) (layer F.Cu) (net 2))
 (segment (start -11.3411 -1.42748) (end -9.999559 -2.769021) (width 0.5) (layer F.Cu) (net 2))
 (segment (start -6.6548 -0.541769) (end -6.6548 -0.7366) (width 0.5) (layer F.Cu) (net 2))
 (via (at -13.63472 -3.15722) (size 0.8) (drill 0.4) (layers F.Cu B.Cu) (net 2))
 (via (at -12.86256 4.25958) (size 0.8) (drill 0.4) (layers F.Cu B.Cu) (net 2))
 (via (at -13.6525 0.8509) (size 0.8) (drill 0.4) (layers F.Cu B.Cu) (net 2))
 (via (at -6.6548 -0.541769) (size 0.8) (drill 0.4) (layers F.Cu B.Cu) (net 2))
 (segment (start -4.445 1.5875) (end -6.574269 -0.541769) (width 0.2) (layer F.Cu) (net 2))
 (segment (start -6.574269 -0.541769) (end -6.6548 -0.541769) (width 0.2) (layer F.Cu) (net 2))
 (via (at -5.85978 1.56464) (size 0.8) (drill 0.4) (layers F.Cu B.Cu) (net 6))
 (segment (start -5.023839 0.728699) (end -5.85978 1.56464) (width 0.2) (layer B.Cu) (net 6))
 (segment (start -6.29412 1.99898) (end -8.32358 1.99898) (width 0.2) (layer F.Cu) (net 6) (status 20))
 (segment (start -5.85978 1.56464) (end -6.29412 1.99898) (width 0.2) (layer F.Cu) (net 6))
 (segment (start -2.763801 0.728699) (end -3.398801 0.728699) (width 0.2) (layer B.Cu) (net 6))
 (segment (start -1.905 1.5875) (end -2.763801 0.728699) (width 0.2) (layer B.Cu) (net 6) (status 10))
 (segment (start -3.398801 0.728699) (end -5.023839 0.728699) (width 0.2) (layer B.Cu) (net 6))
 (segment (start -12.001592 0.922079) (end -12.001592 3.075881) (width 1) (layer F.Cu) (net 7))
 (segment (start -9.59358 -0.54102) (end -10.538493 -0.54102) (width 1) (layer F.Cu) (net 7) (status 10))
 (segment (start -10.538493 -0.54102) (end -12.001592 0.922079) (width 1) (layer F.Cu) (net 7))
 (segment (start -12.001592 3.075881) (end -10.480073 4.5974) (width 1) (layer F.Cu) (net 7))
 (segment (start -0.635 3.647762) (end -0.635 2.8575) (width 1) (layer F.Cu) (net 7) (status 20))
 (segment (start -1.584638 4.5974) (end -0.635 3.647762) (width 1) (layer F.Cu) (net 7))
 (segment (start -10.480073 4.5974) (end -1.584638 4.5974) (width 1) (layer F.Cu) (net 7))
 (segment (start -7.115579 1.218561) (end -7.60516 0.72898) (width 1) (layer B.Cu) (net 3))
 (segment (start -7.115579 2.049947) (end -7.115579 1.218561) (width 1) (layer B.Cu) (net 3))
 (segment (start -5.049225 4.116301) (end -7.115579 2.049947) (width 1) (layer B.Cu) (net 3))
 (segment (start -3.643539 4.116301) (end -5.049225 4.116301) (width 1) (layer B.Cu) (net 3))
 (segment (start -3.175 3.647762) (end -3.643539 4.116301) (width 1) (layer B.Cu) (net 3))
 (segment (start -7.60516 0.72898) (end -8.32358 0.72898) (width 1) (layer B.Cu) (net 3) (status 20))
 (segment (start -3.175 2.8575) (end -3.175 3.647762) (width 1) (layer B.Cu) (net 3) (status 10))
 (segment (start -5.235262 2.8575) (end -5.775151 3.397389) (width 1) (layer F.Cu) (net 1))
 (segment (start -10.801581 2.578821) (end -10.801581 1.419138) (width 1) (layer F.Cu) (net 1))
 (segment (start -10.111423 0.72898) (end -9.59358 0.72898) (width 1) (layer F.Cu) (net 1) (status 20))
 (segment (start -9.983013 3.397389) (end -10.801581 2.578821) (width 1) (layer F.Cu) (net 1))
 (segment (start -5.775151 3.397389) (end -9.983013 3.397389) (width 1) (layer F.Cu) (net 1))
 (segment (start -4.445 2.8575) (end -5.235262 2.8575) (width 1) (layer F.Cu) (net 1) (status 10))
 (segment (start -10.801581 1.419138) (end -10.111423 0.72898) (width 1) (layer F.Cu) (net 1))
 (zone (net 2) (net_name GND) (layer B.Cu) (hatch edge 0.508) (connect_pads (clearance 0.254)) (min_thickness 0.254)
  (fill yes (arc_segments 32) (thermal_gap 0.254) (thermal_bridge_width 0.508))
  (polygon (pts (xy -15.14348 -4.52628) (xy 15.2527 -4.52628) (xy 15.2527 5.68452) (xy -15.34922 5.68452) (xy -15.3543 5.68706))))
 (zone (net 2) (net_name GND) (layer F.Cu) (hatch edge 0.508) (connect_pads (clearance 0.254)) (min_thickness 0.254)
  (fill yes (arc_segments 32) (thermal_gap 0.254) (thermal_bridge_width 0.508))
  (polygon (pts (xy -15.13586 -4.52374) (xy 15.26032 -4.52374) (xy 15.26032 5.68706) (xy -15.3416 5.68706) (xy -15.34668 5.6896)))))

